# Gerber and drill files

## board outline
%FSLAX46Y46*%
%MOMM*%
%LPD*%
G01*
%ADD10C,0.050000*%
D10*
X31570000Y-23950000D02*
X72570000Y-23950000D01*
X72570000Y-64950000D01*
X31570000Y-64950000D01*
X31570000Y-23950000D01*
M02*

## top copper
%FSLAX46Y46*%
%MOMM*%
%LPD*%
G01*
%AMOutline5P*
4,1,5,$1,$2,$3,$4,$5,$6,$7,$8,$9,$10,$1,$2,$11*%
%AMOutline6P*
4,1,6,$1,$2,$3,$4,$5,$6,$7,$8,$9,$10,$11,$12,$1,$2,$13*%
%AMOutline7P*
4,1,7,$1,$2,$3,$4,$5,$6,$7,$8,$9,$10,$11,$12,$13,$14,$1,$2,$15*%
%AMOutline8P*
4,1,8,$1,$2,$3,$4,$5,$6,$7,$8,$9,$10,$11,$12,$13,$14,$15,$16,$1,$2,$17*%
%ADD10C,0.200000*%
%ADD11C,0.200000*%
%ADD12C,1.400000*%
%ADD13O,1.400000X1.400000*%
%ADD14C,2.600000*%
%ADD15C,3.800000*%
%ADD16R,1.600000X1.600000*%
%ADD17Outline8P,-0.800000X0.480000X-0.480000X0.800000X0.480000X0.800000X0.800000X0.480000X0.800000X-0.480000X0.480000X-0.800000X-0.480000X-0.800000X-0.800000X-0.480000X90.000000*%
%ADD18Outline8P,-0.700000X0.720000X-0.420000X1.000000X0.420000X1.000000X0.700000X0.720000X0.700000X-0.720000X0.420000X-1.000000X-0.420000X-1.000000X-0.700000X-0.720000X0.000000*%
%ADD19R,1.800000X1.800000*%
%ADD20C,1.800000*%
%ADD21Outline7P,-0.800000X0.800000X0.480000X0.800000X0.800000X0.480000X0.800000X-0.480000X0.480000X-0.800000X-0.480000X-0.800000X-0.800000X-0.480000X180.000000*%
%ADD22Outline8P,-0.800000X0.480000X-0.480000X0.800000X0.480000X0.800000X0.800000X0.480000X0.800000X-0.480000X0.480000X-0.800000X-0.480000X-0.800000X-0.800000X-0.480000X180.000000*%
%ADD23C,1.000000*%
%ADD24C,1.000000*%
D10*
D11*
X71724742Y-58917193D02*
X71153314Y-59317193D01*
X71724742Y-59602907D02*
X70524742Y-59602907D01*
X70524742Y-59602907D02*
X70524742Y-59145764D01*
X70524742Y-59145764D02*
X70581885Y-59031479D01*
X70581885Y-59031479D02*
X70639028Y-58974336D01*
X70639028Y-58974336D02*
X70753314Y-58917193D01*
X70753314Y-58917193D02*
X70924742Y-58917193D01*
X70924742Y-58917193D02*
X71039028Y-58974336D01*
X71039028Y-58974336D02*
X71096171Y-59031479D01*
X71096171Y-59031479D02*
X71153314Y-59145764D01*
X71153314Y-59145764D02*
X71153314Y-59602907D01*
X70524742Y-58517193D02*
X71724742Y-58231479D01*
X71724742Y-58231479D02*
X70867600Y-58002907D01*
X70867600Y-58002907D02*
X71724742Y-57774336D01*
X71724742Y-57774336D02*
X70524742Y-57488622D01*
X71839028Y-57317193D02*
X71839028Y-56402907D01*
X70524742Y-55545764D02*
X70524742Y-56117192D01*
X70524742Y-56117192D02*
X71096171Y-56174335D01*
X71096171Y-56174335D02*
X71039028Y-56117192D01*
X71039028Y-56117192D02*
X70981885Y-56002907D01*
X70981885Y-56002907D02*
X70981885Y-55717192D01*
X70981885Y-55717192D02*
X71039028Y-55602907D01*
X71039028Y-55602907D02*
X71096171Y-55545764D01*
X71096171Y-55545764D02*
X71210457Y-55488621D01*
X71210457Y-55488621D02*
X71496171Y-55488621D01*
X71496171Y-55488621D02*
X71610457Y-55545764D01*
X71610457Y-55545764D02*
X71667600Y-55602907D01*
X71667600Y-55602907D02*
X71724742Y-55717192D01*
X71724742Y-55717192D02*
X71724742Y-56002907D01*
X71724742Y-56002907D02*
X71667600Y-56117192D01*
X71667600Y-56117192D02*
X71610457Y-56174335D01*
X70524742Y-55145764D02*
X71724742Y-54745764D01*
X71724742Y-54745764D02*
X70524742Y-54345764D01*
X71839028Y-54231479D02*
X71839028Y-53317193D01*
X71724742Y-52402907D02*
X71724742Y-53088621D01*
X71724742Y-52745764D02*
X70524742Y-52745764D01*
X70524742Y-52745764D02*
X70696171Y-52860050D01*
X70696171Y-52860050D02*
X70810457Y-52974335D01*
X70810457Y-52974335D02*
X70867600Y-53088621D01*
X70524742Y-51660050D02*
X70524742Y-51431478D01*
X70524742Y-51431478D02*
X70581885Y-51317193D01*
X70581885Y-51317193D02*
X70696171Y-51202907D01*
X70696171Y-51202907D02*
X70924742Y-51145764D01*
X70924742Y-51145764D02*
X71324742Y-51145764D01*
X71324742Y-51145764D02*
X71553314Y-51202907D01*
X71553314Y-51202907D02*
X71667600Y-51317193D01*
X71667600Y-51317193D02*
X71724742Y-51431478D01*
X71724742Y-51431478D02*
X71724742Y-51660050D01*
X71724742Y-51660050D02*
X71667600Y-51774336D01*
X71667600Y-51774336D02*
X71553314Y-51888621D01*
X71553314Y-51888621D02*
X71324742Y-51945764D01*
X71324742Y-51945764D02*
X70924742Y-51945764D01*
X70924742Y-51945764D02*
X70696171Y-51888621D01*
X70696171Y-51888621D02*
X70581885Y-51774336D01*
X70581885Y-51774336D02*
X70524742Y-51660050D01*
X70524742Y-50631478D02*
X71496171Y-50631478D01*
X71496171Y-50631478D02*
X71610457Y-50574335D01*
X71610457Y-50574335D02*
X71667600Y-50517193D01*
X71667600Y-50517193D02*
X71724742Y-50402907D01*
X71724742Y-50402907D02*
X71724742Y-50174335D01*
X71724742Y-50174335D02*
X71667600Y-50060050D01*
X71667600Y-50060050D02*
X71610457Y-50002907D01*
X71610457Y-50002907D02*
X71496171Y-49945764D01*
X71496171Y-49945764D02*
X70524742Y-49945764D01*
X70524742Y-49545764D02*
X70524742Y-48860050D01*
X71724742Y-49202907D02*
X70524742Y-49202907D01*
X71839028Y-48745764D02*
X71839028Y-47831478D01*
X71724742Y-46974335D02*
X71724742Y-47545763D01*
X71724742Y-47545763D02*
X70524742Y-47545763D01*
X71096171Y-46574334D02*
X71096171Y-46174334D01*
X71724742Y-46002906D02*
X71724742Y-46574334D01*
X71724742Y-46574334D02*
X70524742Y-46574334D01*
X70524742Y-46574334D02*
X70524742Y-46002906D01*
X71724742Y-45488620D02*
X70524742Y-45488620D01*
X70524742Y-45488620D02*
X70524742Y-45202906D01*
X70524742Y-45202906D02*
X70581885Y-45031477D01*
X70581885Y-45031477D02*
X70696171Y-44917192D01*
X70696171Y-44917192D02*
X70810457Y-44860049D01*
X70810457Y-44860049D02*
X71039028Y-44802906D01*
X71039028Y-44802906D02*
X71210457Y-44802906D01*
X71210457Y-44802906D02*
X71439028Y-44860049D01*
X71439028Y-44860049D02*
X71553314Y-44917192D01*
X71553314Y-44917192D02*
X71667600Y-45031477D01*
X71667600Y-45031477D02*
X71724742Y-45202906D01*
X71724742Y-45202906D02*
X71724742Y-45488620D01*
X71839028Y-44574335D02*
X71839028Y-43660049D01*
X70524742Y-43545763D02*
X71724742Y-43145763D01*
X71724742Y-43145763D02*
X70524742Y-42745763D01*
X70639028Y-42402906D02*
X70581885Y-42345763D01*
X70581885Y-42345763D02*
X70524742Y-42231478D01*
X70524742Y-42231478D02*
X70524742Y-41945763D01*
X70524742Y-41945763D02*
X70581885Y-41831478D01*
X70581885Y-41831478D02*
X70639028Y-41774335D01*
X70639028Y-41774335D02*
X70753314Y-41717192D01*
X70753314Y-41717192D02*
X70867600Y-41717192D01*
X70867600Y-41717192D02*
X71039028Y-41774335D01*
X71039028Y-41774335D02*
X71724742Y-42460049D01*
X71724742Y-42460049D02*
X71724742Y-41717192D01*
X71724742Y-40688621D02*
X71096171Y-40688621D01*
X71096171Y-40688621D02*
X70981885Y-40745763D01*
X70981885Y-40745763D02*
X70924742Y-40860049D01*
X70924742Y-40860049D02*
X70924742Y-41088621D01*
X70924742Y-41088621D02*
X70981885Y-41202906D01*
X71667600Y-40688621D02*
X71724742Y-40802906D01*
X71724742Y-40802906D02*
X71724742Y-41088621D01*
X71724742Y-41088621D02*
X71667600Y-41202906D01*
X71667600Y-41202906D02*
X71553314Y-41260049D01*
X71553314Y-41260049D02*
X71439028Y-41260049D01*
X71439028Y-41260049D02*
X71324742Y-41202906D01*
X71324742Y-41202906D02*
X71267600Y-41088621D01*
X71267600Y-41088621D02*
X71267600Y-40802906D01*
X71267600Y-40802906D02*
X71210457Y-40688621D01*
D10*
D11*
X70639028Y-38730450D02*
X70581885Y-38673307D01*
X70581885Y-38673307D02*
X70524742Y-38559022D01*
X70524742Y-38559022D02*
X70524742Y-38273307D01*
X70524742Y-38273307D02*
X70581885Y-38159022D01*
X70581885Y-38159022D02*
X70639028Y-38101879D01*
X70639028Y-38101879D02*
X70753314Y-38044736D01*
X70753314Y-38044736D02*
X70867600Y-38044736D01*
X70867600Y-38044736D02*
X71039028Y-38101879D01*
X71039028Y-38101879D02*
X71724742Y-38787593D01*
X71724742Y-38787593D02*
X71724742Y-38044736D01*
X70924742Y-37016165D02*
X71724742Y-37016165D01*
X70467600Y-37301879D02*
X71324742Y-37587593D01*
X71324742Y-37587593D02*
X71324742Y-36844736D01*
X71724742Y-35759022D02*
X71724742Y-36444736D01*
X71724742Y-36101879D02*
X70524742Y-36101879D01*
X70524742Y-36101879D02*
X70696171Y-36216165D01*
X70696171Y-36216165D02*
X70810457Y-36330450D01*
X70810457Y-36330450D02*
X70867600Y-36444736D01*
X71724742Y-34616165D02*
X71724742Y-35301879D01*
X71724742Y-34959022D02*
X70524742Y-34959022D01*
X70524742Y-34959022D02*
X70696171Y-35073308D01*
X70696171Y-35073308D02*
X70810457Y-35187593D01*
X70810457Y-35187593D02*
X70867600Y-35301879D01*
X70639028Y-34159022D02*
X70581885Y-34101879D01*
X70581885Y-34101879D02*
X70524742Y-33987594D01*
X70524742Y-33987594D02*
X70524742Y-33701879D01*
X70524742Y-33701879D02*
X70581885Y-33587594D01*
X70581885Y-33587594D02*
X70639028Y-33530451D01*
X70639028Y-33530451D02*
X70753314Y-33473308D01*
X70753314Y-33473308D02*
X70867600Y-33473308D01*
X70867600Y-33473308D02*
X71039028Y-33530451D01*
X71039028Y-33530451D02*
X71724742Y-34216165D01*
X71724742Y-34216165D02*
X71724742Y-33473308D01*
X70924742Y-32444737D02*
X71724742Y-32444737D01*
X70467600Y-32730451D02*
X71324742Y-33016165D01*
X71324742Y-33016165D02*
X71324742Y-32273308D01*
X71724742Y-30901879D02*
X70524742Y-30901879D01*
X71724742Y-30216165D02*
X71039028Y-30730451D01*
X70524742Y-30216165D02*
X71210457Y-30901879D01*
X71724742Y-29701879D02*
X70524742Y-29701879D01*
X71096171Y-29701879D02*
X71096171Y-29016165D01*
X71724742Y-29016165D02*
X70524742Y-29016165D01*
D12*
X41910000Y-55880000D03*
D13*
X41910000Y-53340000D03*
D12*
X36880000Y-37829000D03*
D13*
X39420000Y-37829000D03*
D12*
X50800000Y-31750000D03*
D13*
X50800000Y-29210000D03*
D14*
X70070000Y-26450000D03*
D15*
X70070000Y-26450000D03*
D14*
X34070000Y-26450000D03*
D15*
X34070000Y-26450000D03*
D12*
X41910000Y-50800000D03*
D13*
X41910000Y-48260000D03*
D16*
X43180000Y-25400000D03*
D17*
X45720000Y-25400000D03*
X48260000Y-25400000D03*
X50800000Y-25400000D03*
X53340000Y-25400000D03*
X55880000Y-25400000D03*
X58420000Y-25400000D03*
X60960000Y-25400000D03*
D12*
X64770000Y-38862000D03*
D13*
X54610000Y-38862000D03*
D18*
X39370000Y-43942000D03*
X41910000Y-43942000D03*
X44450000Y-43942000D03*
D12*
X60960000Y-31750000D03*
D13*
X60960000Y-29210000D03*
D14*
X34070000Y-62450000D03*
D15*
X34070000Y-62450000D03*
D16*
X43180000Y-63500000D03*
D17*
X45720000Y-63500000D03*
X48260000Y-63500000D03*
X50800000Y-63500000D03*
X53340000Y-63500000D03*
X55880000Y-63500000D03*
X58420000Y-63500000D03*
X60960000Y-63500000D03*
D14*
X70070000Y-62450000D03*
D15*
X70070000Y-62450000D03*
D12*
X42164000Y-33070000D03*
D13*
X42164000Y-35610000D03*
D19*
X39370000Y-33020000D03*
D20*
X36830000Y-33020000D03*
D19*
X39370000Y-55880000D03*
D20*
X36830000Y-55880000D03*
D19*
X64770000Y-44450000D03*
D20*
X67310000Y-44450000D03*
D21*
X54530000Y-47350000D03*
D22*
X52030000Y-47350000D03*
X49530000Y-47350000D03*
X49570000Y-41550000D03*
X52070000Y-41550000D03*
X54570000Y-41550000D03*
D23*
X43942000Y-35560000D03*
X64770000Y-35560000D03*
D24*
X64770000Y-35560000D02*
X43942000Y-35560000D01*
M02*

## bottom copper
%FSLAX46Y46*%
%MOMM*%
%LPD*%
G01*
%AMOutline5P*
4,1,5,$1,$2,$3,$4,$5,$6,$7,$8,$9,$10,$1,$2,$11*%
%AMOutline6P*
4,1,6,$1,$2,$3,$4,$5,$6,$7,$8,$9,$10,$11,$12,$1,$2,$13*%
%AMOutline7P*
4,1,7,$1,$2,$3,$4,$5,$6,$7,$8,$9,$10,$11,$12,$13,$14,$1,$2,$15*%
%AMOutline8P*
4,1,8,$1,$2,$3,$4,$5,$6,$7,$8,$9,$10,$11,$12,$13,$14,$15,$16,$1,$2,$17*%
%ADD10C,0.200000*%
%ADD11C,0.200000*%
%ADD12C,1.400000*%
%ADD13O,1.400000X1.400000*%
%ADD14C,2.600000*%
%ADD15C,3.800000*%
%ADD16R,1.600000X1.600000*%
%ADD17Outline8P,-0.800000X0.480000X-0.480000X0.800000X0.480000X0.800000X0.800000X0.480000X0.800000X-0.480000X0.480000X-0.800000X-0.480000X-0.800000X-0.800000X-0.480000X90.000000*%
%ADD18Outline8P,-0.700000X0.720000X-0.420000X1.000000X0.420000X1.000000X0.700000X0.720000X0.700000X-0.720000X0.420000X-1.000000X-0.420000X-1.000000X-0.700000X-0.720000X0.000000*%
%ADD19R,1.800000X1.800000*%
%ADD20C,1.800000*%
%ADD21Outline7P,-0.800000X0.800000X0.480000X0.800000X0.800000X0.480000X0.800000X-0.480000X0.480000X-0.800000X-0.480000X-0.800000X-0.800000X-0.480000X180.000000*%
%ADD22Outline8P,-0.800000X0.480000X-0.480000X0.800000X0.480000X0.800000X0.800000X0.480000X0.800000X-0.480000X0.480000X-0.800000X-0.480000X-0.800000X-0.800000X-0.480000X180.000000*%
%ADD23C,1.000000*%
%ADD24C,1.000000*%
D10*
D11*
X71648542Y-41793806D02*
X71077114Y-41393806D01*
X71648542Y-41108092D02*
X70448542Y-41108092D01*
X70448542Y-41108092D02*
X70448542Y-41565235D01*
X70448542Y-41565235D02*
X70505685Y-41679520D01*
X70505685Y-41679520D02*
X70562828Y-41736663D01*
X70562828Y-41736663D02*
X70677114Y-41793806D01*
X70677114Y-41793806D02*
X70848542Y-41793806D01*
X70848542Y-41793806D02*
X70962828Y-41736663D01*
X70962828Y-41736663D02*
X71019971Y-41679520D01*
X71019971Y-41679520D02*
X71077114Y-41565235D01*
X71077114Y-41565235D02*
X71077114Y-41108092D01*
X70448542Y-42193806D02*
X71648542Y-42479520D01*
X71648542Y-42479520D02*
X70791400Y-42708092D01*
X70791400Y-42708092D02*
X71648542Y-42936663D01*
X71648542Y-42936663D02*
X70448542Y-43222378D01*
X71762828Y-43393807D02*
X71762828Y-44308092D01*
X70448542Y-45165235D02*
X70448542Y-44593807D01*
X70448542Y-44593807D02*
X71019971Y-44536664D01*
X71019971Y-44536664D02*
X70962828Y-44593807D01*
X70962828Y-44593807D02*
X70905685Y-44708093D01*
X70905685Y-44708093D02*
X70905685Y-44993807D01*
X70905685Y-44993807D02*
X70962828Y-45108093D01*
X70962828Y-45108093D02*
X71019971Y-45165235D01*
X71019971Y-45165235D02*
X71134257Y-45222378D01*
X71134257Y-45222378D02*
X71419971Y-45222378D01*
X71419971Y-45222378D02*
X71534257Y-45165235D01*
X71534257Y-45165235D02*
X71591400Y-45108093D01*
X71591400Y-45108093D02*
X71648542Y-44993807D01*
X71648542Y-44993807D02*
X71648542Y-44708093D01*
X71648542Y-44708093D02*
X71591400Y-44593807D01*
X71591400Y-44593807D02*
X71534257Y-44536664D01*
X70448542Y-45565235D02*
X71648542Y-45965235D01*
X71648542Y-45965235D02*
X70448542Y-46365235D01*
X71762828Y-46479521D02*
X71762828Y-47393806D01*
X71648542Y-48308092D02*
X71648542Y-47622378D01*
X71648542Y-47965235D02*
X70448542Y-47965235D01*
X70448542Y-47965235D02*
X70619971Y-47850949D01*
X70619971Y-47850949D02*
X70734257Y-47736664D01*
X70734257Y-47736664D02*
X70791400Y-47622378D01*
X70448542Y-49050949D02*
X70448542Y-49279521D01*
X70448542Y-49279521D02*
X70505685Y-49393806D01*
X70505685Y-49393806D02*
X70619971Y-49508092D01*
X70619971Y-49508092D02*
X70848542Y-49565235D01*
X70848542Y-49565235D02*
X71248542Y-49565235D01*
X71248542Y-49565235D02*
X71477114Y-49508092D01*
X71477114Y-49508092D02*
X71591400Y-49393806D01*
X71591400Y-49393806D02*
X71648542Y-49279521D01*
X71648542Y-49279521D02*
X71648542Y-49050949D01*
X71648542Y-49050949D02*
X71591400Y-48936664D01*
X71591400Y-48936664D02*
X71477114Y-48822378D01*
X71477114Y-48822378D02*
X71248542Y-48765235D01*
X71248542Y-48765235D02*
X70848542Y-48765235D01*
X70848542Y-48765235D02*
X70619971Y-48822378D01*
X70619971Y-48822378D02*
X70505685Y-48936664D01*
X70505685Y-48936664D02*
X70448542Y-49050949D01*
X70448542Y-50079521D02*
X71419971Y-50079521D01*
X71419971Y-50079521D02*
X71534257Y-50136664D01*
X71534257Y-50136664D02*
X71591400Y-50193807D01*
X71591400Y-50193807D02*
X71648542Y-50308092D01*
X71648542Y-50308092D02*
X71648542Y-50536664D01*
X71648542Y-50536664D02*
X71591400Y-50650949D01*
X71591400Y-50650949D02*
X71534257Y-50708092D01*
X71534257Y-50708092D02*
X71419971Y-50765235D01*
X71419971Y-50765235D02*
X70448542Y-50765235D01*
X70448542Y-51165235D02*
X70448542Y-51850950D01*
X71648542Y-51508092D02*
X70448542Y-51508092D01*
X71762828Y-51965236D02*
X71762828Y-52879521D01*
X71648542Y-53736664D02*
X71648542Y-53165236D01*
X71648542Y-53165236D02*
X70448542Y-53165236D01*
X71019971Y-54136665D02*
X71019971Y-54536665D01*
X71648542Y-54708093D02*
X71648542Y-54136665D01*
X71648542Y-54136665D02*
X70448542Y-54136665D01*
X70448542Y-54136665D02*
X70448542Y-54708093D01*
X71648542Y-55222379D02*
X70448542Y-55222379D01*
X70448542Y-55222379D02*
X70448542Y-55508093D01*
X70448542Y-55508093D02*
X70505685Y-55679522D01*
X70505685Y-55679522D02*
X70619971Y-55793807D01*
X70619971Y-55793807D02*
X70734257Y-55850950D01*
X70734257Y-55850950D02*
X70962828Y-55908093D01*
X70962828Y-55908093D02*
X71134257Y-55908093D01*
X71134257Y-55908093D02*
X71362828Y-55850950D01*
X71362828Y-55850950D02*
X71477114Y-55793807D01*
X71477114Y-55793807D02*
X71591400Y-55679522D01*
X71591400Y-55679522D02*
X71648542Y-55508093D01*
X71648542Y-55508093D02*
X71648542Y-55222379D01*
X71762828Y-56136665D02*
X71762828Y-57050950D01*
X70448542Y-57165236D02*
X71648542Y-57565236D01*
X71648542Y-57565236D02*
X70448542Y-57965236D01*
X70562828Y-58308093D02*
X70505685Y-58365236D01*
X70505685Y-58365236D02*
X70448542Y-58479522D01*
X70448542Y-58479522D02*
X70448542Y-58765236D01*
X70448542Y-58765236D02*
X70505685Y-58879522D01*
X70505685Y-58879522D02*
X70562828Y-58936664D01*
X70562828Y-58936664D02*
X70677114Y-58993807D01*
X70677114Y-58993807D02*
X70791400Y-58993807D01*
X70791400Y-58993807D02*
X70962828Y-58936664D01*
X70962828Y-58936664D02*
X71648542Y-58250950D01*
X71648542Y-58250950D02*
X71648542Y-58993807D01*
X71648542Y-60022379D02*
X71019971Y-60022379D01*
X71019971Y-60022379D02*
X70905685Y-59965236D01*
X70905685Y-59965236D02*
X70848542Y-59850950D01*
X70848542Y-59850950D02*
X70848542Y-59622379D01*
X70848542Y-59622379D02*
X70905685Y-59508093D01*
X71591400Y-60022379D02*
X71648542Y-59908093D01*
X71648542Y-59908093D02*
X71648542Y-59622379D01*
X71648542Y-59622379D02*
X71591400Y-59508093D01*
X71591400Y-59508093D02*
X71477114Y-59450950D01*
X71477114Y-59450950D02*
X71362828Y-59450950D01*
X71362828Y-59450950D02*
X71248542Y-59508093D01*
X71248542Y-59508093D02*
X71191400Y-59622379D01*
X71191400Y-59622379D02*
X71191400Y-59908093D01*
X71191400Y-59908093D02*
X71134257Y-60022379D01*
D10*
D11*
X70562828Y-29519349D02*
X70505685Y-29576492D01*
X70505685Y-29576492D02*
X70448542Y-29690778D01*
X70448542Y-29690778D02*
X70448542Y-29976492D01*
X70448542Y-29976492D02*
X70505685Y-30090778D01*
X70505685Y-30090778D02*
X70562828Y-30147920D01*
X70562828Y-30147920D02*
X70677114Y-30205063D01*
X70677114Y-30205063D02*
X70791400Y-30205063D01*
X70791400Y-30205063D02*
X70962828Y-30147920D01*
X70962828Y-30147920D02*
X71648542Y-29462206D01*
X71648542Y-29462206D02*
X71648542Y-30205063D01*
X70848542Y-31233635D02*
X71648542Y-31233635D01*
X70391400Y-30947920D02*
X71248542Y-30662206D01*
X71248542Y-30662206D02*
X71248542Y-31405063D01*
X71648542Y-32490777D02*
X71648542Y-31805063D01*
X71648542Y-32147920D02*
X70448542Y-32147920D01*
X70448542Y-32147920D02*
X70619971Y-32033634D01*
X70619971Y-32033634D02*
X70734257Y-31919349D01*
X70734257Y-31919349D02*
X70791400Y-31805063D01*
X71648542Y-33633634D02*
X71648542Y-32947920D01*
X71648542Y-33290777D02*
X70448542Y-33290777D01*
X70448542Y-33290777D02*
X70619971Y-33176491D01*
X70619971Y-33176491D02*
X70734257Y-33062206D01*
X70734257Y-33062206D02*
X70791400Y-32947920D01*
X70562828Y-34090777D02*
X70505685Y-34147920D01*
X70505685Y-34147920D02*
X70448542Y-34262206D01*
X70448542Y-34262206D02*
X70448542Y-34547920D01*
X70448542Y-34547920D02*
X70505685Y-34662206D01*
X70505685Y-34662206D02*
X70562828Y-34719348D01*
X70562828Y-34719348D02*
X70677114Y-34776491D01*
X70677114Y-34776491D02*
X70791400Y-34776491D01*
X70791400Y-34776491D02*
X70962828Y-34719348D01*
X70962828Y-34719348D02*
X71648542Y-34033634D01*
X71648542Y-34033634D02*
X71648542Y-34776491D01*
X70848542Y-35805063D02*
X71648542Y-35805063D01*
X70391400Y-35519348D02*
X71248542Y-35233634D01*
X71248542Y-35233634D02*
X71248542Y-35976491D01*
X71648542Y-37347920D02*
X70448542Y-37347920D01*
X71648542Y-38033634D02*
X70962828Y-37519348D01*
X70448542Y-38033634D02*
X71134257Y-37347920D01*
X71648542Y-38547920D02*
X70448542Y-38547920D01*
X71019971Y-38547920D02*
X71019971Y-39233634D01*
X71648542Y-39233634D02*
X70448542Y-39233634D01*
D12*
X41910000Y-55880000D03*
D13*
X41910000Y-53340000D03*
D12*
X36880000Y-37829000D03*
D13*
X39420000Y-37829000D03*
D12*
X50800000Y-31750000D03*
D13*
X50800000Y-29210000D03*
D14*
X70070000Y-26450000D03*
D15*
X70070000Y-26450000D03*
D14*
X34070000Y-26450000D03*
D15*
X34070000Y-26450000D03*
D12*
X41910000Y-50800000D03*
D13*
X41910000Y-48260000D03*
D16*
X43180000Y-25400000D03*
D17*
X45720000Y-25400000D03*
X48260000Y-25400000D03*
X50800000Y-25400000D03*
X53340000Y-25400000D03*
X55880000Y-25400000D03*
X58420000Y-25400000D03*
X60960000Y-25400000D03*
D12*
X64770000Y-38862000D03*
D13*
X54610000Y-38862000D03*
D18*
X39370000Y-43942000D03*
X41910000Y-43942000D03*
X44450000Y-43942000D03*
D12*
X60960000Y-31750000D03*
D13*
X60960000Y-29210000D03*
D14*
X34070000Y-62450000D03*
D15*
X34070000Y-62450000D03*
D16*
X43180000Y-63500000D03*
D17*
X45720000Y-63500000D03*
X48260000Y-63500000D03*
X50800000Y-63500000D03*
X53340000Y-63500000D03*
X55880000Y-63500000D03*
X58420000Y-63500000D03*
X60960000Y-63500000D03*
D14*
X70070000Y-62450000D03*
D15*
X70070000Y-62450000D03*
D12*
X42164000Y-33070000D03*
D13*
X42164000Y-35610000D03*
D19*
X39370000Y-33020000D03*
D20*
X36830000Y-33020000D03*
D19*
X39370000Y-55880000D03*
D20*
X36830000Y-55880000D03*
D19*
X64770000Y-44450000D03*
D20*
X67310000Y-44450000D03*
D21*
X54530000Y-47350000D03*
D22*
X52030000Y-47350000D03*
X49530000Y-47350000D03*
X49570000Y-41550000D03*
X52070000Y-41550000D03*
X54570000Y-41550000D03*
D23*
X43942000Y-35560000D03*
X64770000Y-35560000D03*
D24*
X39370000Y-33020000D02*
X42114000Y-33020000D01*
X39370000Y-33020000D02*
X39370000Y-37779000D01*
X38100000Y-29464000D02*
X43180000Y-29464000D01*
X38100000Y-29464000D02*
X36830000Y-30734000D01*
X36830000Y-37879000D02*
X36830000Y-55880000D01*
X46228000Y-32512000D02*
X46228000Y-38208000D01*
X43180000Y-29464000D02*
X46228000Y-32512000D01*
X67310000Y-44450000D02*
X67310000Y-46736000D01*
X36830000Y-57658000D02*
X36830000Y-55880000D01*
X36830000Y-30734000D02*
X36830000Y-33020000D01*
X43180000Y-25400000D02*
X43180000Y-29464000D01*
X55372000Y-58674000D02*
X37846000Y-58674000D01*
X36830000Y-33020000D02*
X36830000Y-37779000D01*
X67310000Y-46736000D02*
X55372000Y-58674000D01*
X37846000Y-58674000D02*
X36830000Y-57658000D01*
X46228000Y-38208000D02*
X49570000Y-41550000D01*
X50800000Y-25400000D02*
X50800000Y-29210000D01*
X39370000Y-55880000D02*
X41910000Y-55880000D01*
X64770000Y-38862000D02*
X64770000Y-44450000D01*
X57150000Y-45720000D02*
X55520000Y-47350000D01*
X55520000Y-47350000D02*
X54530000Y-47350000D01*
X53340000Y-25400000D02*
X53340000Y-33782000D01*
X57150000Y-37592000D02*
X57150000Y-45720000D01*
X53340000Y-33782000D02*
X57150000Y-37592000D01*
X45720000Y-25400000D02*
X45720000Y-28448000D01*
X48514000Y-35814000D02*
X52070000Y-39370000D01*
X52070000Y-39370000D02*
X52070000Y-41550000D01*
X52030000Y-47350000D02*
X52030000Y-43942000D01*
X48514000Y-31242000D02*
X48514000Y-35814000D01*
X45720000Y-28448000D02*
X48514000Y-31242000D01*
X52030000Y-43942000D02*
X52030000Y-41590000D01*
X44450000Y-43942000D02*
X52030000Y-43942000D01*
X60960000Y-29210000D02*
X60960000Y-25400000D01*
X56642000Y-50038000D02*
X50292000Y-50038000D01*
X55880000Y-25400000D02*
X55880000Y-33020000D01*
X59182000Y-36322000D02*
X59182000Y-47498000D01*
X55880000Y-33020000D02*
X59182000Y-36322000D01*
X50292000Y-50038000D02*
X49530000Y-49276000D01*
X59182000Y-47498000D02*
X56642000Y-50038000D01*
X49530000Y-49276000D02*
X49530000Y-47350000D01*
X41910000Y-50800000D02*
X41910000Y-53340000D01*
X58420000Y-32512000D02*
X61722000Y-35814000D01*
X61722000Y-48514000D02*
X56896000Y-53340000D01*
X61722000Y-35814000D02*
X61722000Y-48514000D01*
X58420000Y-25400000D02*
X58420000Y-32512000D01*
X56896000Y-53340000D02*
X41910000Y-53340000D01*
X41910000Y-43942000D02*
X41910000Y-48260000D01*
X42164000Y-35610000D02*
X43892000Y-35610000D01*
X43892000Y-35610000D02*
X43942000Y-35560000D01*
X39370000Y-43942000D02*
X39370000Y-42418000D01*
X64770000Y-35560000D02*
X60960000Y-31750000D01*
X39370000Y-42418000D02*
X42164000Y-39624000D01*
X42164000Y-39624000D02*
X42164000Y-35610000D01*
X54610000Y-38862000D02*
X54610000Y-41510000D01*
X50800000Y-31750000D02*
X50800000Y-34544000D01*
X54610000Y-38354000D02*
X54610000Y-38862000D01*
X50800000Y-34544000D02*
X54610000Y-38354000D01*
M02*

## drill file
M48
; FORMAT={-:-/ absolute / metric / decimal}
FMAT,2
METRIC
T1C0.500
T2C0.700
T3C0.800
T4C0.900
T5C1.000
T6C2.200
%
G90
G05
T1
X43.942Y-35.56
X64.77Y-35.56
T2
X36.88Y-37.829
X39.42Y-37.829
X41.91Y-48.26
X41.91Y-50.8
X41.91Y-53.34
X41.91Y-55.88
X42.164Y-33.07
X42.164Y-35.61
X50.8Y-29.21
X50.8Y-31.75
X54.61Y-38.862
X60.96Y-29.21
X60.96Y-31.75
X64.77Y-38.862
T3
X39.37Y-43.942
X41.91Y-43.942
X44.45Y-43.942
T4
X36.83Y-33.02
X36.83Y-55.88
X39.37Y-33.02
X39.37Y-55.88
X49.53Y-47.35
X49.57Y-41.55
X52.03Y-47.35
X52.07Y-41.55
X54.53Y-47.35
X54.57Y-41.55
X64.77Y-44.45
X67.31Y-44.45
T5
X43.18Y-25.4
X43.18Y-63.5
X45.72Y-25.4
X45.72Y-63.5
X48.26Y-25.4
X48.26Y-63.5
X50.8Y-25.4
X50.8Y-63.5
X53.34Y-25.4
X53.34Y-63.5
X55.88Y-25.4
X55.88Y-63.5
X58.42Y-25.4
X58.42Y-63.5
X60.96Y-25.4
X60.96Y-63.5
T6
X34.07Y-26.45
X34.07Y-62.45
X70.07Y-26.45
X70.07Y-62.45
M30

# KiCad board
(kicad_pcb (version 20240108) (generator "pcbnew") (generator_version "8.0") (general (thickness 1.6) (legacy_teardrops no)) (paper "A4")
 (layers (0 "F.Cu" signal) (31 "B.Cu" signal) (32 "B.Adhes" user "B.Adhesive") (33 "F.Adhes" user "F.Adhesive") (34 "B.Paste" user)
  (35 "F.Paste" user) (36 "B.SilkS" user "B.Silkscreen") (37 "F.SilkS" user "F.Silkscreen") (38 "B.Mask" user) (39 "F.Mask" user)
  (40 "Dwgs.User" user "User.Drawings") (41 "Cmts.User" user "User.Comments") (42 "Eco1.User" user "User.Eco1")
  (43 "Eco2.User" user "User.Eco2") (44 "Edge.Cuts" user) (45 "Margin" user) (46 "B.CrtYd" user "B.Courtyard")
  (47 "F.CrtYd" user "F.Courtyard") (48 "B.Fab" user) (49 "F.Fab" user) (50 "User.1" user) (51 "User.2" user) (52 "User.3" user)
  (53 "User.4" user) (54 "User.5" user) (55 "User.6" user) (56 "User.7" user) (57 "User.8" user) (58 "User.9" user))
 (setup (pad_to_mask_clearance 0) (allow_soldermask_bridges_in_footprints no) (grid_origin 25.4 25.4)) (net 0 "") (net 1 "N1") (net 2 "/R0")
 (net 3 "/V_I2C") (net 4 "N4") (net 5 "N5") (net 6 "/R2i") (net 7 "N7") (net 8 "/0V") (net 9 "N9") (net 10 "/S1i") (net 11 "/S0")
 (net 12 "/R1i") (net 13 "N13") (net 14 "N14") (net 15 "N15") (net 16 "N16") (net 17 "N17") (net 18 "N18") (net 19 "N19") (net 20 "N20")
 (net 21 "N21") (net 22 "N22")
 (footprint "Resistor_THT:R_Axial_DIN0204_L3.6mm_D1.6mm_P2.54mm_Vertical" (layer "F.Cu") (at 41.91 55.88 90)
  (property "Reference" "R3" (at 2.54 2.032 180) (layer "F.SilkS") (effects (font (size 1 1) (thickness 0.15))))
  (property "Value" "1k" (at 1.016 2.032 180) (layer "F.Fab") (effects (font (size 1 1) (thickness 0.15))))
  (pad "1" thru_hole circle (at 0 0 90) (size 1.4 1.4) (drill 0.7) (layers "*.Cu" "*.Mask") (remove_unused_layers no) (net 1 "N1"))
  (pad "2" thru_hole oval (at 2.54 0 90) (size 1.4 1.4) (drill 0.7) (layers "*.Cu" "*.Mask") (remove_unused_layers no) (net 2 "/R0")))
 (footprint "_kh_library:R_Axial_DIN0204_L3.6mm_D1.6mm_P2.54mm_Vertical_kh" (layer "F.Cu") (at 36.88 37.829)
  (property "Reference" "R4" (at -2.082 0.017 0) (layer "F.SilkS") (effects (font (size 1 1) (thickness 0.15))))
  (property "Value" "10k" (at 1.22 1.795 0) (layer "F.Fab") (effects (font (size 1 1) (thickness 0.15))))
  (pad "1" thru_hole circle (at 0 0) (size 1.4 1.4) (drill 0.7) (layers "*.Cu" "*.Mask") (remove_unused_layers no) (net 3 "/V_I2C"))
  (pad "2" thru_hole oval (at 2.54 0) (size 1.4 1.4) (drill 0.7) (layers "*.Cu" "*.Mask") (remove_unused_layers no) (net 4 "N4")))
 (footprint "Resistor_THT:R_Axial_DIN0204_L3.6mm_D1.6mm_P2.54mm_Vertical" (layer "F.Cu") (at 50.8 31.75 90)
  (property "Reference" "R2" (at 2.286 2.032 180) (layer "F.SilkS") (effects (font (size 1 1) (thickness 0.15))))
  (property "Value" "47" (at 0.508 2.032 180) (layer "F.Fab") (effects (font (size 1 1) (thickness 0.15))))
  (pad "1" thru_hole circle (at 0 0 90) (size 1.4 1.4) (drill 0.7) (layers "*.Cu" "*.Mask") (remove_unused_layers no) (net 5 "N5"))
  (pad "2" thru_hole oval (at 2.54 0 90) (size 1.4 1.4) (drill 0.7) (layers "*.Cu" "*.Mask") (remove_unused_layers no) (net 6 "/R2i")))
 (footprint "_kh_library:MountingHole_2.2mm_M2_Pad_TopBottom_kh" (layer "F.Cu") (at 70.07 26.45)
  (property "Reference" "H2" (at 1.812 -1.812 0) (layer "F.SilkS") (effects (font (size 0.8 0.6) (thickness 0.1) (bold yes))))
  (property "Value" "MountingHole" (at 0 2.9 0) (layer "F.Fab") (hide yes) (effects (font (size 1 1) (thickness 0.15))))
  (pad "1" thru_hole circle (at 0 0) (size 2.6 2.6) (drill 2.2) (layers "*.Cu" "*.Mask") (remove_unused_layers no))
  (pad "1" connect circle (at 0 0) (size 3.8 3.8) (layers "F.Cu" "F.Mask"))
  (pad "1" connect circle (at 0 0) (size 3.8 3.8) (layers "B.Cu" "B.Mask")))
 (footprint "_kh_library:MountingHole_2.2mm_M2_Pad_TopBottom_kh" (layer "F.Cu") (at 34.07 26.45)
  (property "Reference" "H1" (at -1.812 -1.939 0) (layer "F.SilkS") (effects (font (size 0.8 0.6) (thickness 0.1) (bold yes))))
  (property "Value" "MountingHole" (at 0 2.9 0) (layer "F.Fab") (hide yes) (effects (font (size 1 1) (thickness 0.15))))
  (pad "1" thru_hole circle (at 0 0) (size 2.6 2.6) (drill 2.2) (layers "*.Cu" "*.Mask") (remove_unused_layers no))
  (pad "1" connect circle (at 0 0) (size 3.8 3.8) (layers "F.Cu" "F.Mask"))
  (pad "1" connect circle (at 0 0) (size 3.8 3.8) (layers "B.Cu" "B.Mask")))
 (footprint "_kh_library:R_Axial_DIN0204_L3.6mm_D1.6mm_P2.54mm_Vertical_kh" (layer "F.Cu") (at 41.91 50.8 90)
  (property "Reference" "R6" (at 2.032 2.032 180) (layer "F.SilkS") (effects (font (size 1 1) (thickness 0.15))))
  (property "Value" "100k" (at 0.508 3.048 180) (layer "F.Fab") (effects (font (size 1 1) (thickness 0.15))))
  (pad "1" thru_hole circle (at 0 0 90) (size 1.4 1.4) (drill 0.7) (layers "*.Cu" "*.Mask") (remove_unused_layers no) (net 2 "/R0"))
  (pad "2" thru_hole oval (at 2.54 0 90) (size 1.4 1.4) (drill 0.7) (layers "*.Cu" "*.Mask") (remove_unused_layers no) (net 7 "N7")))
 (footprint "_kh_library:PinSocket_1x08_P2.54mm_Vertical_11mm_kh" (layer "F.Cu") (at 43.18 25.4 90)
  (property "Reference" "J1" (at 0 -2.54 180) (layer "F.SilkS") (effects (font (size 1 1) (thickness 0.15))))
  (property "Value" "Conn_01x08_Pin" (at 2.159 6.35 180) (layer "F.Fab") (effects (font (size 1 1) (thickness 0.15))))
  (pad "1" thru_hole rect (at 0 0 90) (size 1.6 1.6) (drill 1) (layers "*.Cu" "*.Mask") (remove_unused_layers no) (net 3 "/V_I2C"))
  (pad "2" thru_hole roundrect (at 0 2.54 90) (size 1.6 1.6) (drill 1) (layers "*.Cu" "*.Mask") (remove_unused_layers no)
   (roundrect_rratio 0) (chamfer_ratio 0.2) (chamfer top_left top_right bottom_left bottom_right) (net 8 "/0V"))
  (pad "3" thru_hole roundrect (at 0 5.08 90) (size 1.6 1.6) (drill 1) (layers "*.Cu" "*.Mask") (remove_unused_layers no)
   (roundrect_rratio 0) (chamfer_ratio 0.2) (chamfer top_left top_right bottom_left bottom_right) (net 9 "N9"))
  (pad "4" thru_hole roundrect (at 0 7.62 90) (size 1.6 1.6) (drill 1) (layers "*.Cu" "*.Mask") (remove_unused_layers no)
   (roundrect_rratio 0) (chamfer_ratio 0.2) (chamfer top_left top_right bottom_left bottom_right) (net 6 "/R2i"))
  (pad "5" thru_hole roundrect (at 0 10.16 90) (size 1.6 1.6) (drill 1) (layers "*.Cu" "*.Mask") (remove_unused_layers no)
   (roundrect_rratio 0) (chamfer_ratio 0.2) (chamfer top_left top_right bottom_left bottom_right) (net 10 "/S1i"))
  (pad "6" thru_hole roundrect (at 0 12.7 90) (size 1.6 1.6) (drill 1) (layers "*.Cu" "*.Mask") (remove_unused_layers no)
   (roundrect_rratio 0) (chamfer_ratio 0.2) (chamfer top_left top_right bottom_left bottom_right) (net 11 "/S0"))
  (pad "7" thru_hole roundrect (at 0 15.24 90) (size 1.6 1.6) (drill 1) (layers "*.Cu" "*.Mask") (remove_unused_layers no)
   (roundrect_rratio 0) (chamfer_ratio 0.2) (chamfer top_left top_right bottom_left bottom_right) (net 2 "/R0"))
  (pad "8" thru_hole roundrect (at 0 17.78 90) (size 1.6 1.6) (drill 1) (layers "*.Cu" "*.Mask") (remove_unused_layers no)
   (roundrect_rratio 0) (chamfer_ratio 0.2) (chamfer top_left top_right bottom_left bottom_right) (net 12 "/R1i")))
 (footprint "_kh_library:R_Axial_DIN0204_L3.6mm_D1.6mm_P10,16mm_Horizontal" (layer "F.Cu") (at 64.77 38.862 180)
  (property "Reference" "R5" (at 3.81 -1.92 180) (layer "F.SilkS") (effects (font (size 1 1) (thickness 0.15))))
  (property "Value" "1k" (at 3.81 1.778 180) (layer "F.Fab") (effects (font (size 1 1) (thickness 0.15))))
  (pad "1" thru_hole circle (at 0 0 180) (size 1.4 1.4) (drill 0.7) (layers "*.Cu" "*.Mask") (remove_unused_layers no) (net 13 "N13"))
  (pad "2" thru_hole oval (at 10.16 0 180) (size 1.4 1.4) (drill 0.7) (layers "*.Cu" "*.Mask") (remove_unused_layers no) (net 5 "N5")))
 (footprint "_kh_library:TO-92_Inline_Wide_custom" (layer "F.Cu") (at 39.37 43.942)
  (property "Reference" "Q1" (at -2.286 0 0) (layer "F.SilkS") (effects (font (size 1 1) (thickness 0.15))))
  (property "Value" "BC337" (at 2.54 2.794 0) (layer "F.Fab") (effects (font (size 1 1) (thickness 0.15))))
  (pad "1" thru_hole roundrect (at 0 0) (size 1.4 2) (drill 0.8) (layers "*.Cu" "*.Mask") (remove_unused_layers no) (roundrect_rratio 0)
   (chamfer_ratio 0.2) (chamfer top_left top_right bottom_left bottom_right) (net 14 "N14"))
  (pad "2" thru_hole roundrect (at 2.54 0) (size 1.4 2) (drill 0.8) (layers "*.Cu" "*.Mask") (remove_unused_layers no) (roundrect_rratio 0)
   (chamfer_ratio 0.2) (chamfer top_left top_right bottom_left bottom_right) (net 7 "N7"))
  (pad "3" thru_hole roundrect (at 5.08 0) (size 1.4 2) (drill 0.8) (layers "*.Cu" "*.Mask") (remove_unused_layers no) (roundrect_rratio 0)
   (chamfer_ratio 0.2) (chamfer top_left top_right bottom_left bottom_right) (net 8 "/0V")))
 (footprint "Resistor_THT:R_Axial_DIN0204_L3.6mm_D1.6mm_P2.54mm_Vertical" (layer "F.Cu") (at 60.96 31.75 90)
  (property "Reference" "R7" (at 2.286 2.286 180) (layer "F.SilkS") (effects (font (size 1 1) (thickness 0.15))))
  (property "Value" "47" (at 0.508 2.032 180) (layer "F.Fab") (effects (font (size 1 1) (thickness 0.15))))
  (pad "1" thru_hole circle (at 0 0 90) (size 1.4 1.4) (drill 0.7) (layers "*.Cu" "*.Mask") (remove_unused_layers no) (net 14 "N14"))
  (pad "2" thru_hole oval (at 2.54 0 90) (size 1.4 1.4) (drill 0.7) (layers "*.Cu" "*.Mask") (remove_unused_layers no) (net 12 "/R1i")))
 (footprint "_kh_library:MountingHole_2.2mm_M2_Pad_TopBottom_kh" (layer "F.Cu") (at 34.07 62.45)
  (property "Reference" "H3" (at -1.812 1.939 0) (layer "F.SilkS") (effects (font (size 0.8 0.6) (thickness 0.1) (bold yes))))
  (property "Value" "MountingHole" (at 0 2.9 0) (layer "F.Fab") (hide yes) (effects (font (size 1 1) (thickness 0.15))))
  (pad "1" thru_hole circle (at 0 0) (size 2.6 2.6) (drill 2.2) (layers "*.Cu" "*.Mask") (remove_unused_layers no))
  (pad "1" connect circle (at 0 0) (size 3.8 3.8) (layers "F.Cu" "F.Mask"))
  (pad "1" connect circle (at 0 0) (size 3.8 3.8) (layers "B.Cu" "B.Mask")))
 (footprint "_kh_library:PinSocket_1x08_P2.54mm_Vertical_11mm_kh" (layer "F.Cu") (at 43.18 63.5 90)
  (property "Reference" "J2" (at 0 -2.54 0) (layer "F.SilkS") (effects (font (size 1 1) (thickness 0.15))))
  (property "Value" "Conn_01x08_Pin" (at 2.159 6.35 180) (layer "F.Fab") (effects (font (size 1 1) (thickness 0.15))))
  (pad "1" thru_hole rect (at 0 0 90) (size 1.6 1.6) (drill 1) (layers "*.Cu" "*.Mask") (remove_unused_layers no) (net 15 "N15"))
  (pad "2" thru_hole roundrect (at 0 2.54 90) (size 1.6 1.6) (drill 1) (layers "*.Cu" "*.Mask") (remove_unused_layers no)
   (roundrect_rratio 0) (chamfer_ratio 0.2) (chamfer top_left top_right bottom_left bottom_right) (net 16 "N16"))
  (pad "3" thru_hole roundrect (at 0 5.08 90) (size 1.6 1.6) (drill 1) (layers "*.Cu" "*.Mask") (remove_unused_layers no)
   (roundrect_rratio 0) (chamfer_ratio 0.2) (chamfer top_left top_right bottom_left bottom_right) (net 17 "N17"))
  (pad "4" thru_hole roundrect (at 0 7.62 90) (size 1.6 1.6) (drill 1) (layers "*.Cu" "*.Mask") (remove_unused_layers no)
   (roundrect_rratio 0) (chamfer_ratio 0.2) (chamfer top_left top_right bottom_left bottom_right) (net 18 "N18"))
  (pad "5" thru_hole roundrect (at 0 10.16 90) (size 1.6 1.6) (drill 1) (layers "*.Cu" "*.Mask") (remove_unused_layers no)
   (roundrect_rratio 0) (chamfer_ratio 0.2) (chamfer top_left top_right bottom_left bottom_right) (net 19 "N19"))
  (pad "6" thru_hole roundrect (at 0 12.7 90) (size 1.6 1.6) (drill 1) (layers "*.Cu" "*.Mask") (remove_unused_layers no)
   (roundrect_rratio 0) (chamfer_ratio 0.2) (chamfer top_left top_right bottom_left bottom_right) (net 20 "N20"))
  (pad "7" thru_hole roundrect (at 0 15.24 90) (size 1.6 1.6) (drill 1) (layers "*.Cu" "*.Mask") (remove_unused_layers no)
   (roundrect_rratio 0) (chamfer_ratio 0.2) (chamfer top_left top_right bottom_left bottom_right) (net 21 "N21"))
  (pad "8" thru_hole roundrect (at 0 17.78 90) (size 1.6 1.6) (drill 1) (layers "*.Cu" "*.Mask") (remove_unused_layers no)
   (roundrect_rratio 0) (chamfer_ratio 0.2) (chamfer top_left top_right bottom_left bottom_right) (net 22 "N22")))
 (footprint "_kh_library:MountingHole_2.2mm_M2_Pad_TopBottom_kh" (layer "F.Cu") (at 70.07 62.45)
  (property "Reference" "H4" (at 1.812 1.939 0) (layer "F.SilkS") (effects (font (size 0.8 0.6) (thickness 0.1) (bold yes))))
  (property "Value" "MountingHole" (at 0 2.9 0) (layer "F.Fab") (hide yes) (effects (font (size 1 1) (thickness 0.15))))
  (pad "1" thru_hole circle (at 0 0) (size 2.6 2.6) (drill 2.2) (layers "*.Cu" "*.Mask") (remove_unused_layers no))
  (pad "1" connect circle (at 0 0) (size 3.8 3.8) (layers "F.Cu" "F.Mask"))
  (pad "1" connect circle (at 0 0) (size 3.8 3.8) (layers "B.Cu" "B.Mask")))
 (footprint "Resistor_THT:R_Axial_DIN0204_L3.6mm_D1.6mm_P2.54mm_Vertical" (layer "F.Cu") (at 42.164 33.07 -90)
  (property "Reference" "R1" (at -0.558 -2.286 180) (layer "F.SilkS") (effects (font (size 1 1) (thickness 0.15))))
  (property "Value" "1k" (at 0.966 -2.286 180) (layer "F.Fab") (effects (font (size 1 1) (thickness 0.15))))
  (pad "1" thru_hole circle (at 0 0 270) (size 1.4 1.4) (drill 0.7) (layers "*.Cu" "*.Mask") (remove_unused_layers no) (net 4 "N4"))
  (pad "2" thru_hole oval (at 2.54 0 270) (size 1.4 1.4) (drill 0.7) (layers "*.Cu" "*.Mask") (remove_unused_layers no) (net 14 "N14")))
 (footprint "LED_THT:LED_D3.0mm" (layer "B.Cu") (at 39.37 33.02 180)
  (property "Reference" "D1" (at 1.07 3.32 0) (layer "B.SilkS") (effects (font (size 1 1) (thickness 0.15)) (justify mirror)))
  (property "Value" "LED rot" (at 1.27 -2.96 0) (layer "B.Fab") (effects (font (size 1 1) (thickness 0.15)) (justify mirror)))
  (pad "1" thru_hole rect (at 0 0 180) (size 1.8 1.8) (drill 0.9) (layers "*.Cu" "*.Mask") (remove_unused_layers no) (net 4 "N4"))
  (pad "2" thru_hole circle (at 2.54 0 180) (size 1.8 1.8) (drill 0.9) (layers "*.Cu" "*.Mask") (remove_unused_layers no) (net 3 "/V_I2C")))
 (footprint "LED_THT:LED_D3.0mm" (layer "B.Cu") (at 39.37 55.88 180)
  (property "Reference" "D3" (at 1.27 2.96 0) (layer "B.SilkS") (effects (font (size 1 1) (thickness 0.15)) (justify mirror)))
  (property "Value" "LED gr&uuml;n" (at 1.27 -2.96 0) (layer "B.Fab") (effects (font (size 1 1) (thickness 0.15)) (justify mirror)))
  (pad "1" thru_hole rect (at 0 0 180) (size 1.8 1.8) (drill 0.9) (layers "*.Cu" "*.Mask") (remove_unused_layers no) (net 1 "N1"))
  (pad "2" thru_hole circle (at 2.54 0 180) (size 1.8 1.8) (drill 0.9) (layers "*.Cu" "*.Mask") (remove_unused_layers no) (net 3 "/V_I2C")))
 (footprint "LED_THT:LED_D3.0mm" (layer "B.Cu") (at 64.77 44.45)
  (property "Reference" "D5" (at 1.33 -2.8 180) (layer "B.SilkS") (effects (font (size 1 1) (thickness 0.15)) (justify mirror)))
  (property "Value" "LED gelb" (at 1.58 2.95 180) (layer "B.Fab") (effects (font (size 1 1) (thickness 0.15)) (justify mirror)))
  (pad "1" thru_hole rect (at 0 0) (size 1.8 1.8) (drill 0.9) (layers "*.Cu" "*.Mask") (remove_unused_layers no) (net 13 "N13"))
  (pad "2" thru_hole circle (at 2.54 0) (size 1.8 1.8) (drill 0.9) (layers "*.Cu" "*.Mask") (remove_unused_layers no) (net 3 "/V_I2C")))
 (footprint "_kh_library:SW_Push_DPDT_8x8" (layer "B.Cu") (at 54.57 47.35 180)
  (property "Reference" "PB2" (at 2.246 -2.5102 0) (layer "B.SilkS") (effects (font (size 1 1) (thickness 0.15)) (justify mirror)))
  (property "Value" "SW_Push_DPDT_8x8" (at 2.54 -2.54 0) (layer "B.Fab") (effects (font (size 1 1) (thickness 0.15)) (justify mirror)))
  (pad "1" thru_hole roundrect (at 0.04 0 180) (size 1.6 1.6) (drill 0.9) (layers "*.Cu" "*.Mask") (remove_unused_layers no)
   (roundrect_rratio 0) (chamfer_ratio 0.2) (chamfer top_right bottom_left bottom_right) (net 10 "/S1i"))
  (pad "2" thru_hole roundrect (at 2.54 0 180) (size 1.6 1.6) (drill 0.9) (layers "*.Cu" "*.Mask") (remove_unused_layers no)
   (roundrect_rratio 0) (chamfer_ratio 0.2) (chamfer top_left top_right bottom_left bottom_right) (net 8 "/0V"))
  (pad "3" thru_hole roundrect (at 5.04 0 180) (size 1.6 1.6) (drill 0.9) (layers "*.Cu" "*.Mask") (remove_unused_layers no)
   (roundrect_rratio 0) (chamfer_ratio 0.2) (chamfer top_left top_right bottom_left bottom_right) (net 11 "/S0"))
  (pad "4" thru_hole roundrect (at 5 5.8 180) (size 1.6 1.6) (drill 0.9) (layers "*.Cu" "*.Mask") (remove_unused_layers no)
   (roundrect_rratio 0) (chamfer_ratio 0.2) (chamfer top_left top_right bottom_left bottom_right) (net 3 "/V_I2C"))
  (pad "5" thru_hole roundrect (at 2.5 5.8 180) (size 1.6 1.6) (drill 0.9) (layers "*.Cu" "*.Mask") (remove_unused_layers no)
   (roundrect_rratio 0) (chamfer_ratio 0.2) (chamfer top_left top_right bottom_left bottom_right) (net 8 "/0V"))
  (pad "6" thru_hole roundrect (at 0 5.8 180) (size 1.6 1.6) (drill 0.9) (layers "*.Cu" "*.Mask") (remove_unused_layers no)
   (roundrect_rratio 0) (chamfer_ratio 0.2) (chamfer top_left top_right bottom_left bottom_right) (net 5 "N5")))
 (gr_rect (start 31.57 23.95) (end 72.57 64.95) (stroke (width 0.05) (type default)) (fill none) (layer "Edge.Cuts"))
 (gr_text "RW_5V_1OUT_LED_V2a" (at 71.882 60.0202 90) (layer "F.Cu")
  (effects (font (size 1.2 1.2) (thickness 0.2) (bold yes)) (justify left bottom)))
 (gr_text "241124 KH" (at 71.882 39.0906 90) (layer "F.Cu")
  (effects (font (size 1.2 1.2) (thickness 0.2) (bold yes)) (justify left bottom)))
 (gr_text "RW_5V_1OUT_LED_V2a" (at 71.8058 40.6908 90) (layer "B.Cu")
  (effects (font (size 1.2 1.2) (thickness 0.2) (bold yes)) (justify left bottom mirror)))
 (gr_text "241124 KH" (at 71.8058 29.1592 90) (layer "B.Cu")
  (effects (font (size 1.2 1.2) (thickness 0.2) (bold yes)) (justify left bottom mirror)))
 (segment (start 39.37 33.02) (end 42.114 33.02) (width 1) (layer "B.Cu") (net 4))
 (segment (start 39.37 33.02) (end 39.37 37.779) (width 1) (layer "B.Cu") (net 4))
 (segment (start 38.1 29.464) (end 43.18 29.464) (width 1) (layer "B.Cu") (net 3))
 (segment (start 38.1 29.464) (end 36.83 30.734) (width 1) (layer "B.Cu") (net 3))
 (segment (start 36.83 37.879) (end 36.83 55.88) (width 1) (layer "B.Cu") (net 3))
 (segment (start 46.228 32.512) (end 46.228 38.208) (width 1) (layer "B.Cu") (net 3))
 (segment (start 43.18 29.464) (end 46.228 32.512) (width 1) (layer "B.Cu") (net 3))
 (segment (start 67.31 44.45) (end 67.31 46.736) (width 1) (layer "B.Cu") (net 3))
 (segment (start 36.83 57.658) (end 36.83 55.88) (width 1) (layer "B.Cu") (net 3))
 (segment (start 36.83 30.734) (end 36.83 33.02) (width 1) (layer "B.Cu") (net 3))
 (segment (start 43.18 25.4) (end 43.18 29.464) (width 1) (layer "B.Cu") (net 3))
 (segment (start 55.372 58.674) (end 37.846 58.674) (width 1) (layer "B.Cu") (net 3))
 (segment (start 36.83 33.02) (end 36.83 37.779) (width 1) (layer "B.Cu") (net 3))
 (segment (start 67.31 46.736) (end 55.372 58.674) (width 1) (layer "B.Cu") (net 3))
 (segment (start 37.846 58.674) (end 36.83 57.658) (width 1) (layer "B.Cu") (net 3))
 (segment (start 46.228 38.208) (end 49.57 41.55) (width 1) (layer "B.Cu") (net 3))
 (segment (start 50.8 25.4) (end 50.8 29.21) (width 1) (layer "B.Cu") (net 6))
 (segment (start 39.37 55.88) (end 41.91 55.88) (width 1) (layer "B.Cu") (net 1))
 (segment (start 64.77 38.862) (end 64.77 44.45) (width 1) (layer "B.Cu") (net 13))
 (segment (start 57.15 45.72) (end 55.52 47.35) (width 1) (layer "B.Cu") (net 10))
 (segment (start 55.52 47.35) (end 54.53 47.35) (width 1) (layer "B.Cu") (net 10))
 (segment (start 53.34 25.4) (end 53.34 33.782) (width 1) (layer "B.Cu") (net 10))
 (segment (start 57.15 37.592) (end 57.15 45.72) (width 1) (layer "B.Cu") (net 10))
 (segment (start 53.34 33.782) (end 57.15 37.592) (width 1) (layer "B.Cu") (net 10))
 (segment (start 45.72 25.4) (end 45.72 28.448) (width 1) (layer "B.Cu") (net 8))
 (segment (start 48.514 35.814) (end 52.07 39.37) (width 1) (layer "B.Cu") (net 8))
 (segment (start 52.07 39.37) (end 52.07 41.55) (width 1) (layer "B.Cu") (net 8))
 (segment (start 52.03 47.35) (end 52.03 43.942) (width 1) (layer "B.Cu") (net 8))
 (segment (start 48.514 31.242) (end 48.514 35.814) (width 1) (layer "B.Cu") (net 8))
 (segment (start 45.72 28.448) (end 48.514 31.242) (width 1) (layer "B.Cu") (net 8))
 (segment (start 52.03 43.942) (end 52.03 41.59) (width 1) (layer "B.Cu") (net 8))
 (segment (start 44.45 43.942) (end 52.03 43.942) (width 1) (layer "B.Cu") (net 8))
 (segment (start 60.96 29.21) (end 60.96 25.4) (width 1) (layer "B.Cu") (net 12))
 (segment (start 56.642 50.038) (end 50.292 50.038) (width 1) (layer "B.Cu") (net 11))
 (segment (start 55.88 25.4) (end 55.88 33.02) (width 1) (layer "B.Cu") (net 11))
 (segment (start 59.182 36.322) (end 59.182 47.498) (width 1) (layer "B.Cu") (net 11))
 (segment (start 55.88 33.02) (end 59.182 36.322) (width 1) (layer "B.Cu") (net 11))
 (segment (start 50.292 50.038) (end 49.53 49.276) (width 1) (layer "B.Cu") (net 11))
 (segment (start 59.182 47.498) (end 56.642 50.038) (width 1) (layer "B.Cu") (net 11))
 (segment (start 49.53 49.276) (end 49.53 47.35) (width 1) (layer "B.Cu") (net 11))
 (segment (start 41.91 50.8) (end 41.91 53.34) (width 1) (layer "B.Cu") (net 2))
 (segment (start 58.42 32.512) (end 61.722 35.814) (width 1) (layer "B.Cu") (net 2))
 (segment (start 61.722 48.514) (end 56.896 53.34) (width 1) (layer "B.Cu") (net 2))
 (segment (start 61.722 35.814) (end 61.722 48.514) (width 1) (layer "B.Cu") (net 2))
 (segment (start 58.42 25.4) (end 58.42 32.512) (width 1) (layer "B.Cu") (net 2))
 (segment (start 56.896 53.34) (end 41.91 53.34) (width 1) (layer "B.Cu") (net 2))
 (segment (start 41.91 43.942) (end 41.91 48.26) (width 1) (layer "B.Cu") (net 7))
 (segment (start 64.77 35.56) (end 43.942 35.56) (width 1) (layer "F.Cu") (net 14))
 (via (at 43.942 35.56) (size 1) (drill 0.5) (layers "F.Cu" "B.Cu") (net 14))
 (via (at 64.77 35.56) (size 1) (drill 0.5) (layers "F.Cu" "B.Cu") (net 14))
 (segment (start 42.164 35.61) (end 43.892 35.61) (width 1) (layer "B.Cu") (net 14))
 (segment (start 43.892 35.61) (end 43.942 35.56) (width 1) (layer "B.Cu") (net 14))
 (segment (start 39.37 43.942) (end 39.37 42.418) (width 1) (layer "B.Cu") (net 14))
 (segment (start 64.77 35.56) (end 60.96 31.75) (width 1) (layer "B.Cu") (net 14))
 (segment (start 39.37 42.418) (end 42.164 39.624) (width 1) (layer "B.Cu") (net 14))
 (segment (start 42.164 39.624) (end 42.164 35.61) (width 1) (layer "B.Cu") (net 14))
 (segment (start 54.61 38.862) (end 54.61 41.51) (width 1) (layer "B.Cu") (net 5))
 (segment (start 50.8 31.75) (end 50.8 34.544) (width 1) (layer "B.Cu") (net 5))
 (segment (start 54.61 38.354) (end 54.61 38.862) (width 1) (layer "B.Cu") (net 5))
 (segment (start 50.8 34.544) (end 54.61 38.354) (width 1) (layer "B.Cu") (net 5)))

